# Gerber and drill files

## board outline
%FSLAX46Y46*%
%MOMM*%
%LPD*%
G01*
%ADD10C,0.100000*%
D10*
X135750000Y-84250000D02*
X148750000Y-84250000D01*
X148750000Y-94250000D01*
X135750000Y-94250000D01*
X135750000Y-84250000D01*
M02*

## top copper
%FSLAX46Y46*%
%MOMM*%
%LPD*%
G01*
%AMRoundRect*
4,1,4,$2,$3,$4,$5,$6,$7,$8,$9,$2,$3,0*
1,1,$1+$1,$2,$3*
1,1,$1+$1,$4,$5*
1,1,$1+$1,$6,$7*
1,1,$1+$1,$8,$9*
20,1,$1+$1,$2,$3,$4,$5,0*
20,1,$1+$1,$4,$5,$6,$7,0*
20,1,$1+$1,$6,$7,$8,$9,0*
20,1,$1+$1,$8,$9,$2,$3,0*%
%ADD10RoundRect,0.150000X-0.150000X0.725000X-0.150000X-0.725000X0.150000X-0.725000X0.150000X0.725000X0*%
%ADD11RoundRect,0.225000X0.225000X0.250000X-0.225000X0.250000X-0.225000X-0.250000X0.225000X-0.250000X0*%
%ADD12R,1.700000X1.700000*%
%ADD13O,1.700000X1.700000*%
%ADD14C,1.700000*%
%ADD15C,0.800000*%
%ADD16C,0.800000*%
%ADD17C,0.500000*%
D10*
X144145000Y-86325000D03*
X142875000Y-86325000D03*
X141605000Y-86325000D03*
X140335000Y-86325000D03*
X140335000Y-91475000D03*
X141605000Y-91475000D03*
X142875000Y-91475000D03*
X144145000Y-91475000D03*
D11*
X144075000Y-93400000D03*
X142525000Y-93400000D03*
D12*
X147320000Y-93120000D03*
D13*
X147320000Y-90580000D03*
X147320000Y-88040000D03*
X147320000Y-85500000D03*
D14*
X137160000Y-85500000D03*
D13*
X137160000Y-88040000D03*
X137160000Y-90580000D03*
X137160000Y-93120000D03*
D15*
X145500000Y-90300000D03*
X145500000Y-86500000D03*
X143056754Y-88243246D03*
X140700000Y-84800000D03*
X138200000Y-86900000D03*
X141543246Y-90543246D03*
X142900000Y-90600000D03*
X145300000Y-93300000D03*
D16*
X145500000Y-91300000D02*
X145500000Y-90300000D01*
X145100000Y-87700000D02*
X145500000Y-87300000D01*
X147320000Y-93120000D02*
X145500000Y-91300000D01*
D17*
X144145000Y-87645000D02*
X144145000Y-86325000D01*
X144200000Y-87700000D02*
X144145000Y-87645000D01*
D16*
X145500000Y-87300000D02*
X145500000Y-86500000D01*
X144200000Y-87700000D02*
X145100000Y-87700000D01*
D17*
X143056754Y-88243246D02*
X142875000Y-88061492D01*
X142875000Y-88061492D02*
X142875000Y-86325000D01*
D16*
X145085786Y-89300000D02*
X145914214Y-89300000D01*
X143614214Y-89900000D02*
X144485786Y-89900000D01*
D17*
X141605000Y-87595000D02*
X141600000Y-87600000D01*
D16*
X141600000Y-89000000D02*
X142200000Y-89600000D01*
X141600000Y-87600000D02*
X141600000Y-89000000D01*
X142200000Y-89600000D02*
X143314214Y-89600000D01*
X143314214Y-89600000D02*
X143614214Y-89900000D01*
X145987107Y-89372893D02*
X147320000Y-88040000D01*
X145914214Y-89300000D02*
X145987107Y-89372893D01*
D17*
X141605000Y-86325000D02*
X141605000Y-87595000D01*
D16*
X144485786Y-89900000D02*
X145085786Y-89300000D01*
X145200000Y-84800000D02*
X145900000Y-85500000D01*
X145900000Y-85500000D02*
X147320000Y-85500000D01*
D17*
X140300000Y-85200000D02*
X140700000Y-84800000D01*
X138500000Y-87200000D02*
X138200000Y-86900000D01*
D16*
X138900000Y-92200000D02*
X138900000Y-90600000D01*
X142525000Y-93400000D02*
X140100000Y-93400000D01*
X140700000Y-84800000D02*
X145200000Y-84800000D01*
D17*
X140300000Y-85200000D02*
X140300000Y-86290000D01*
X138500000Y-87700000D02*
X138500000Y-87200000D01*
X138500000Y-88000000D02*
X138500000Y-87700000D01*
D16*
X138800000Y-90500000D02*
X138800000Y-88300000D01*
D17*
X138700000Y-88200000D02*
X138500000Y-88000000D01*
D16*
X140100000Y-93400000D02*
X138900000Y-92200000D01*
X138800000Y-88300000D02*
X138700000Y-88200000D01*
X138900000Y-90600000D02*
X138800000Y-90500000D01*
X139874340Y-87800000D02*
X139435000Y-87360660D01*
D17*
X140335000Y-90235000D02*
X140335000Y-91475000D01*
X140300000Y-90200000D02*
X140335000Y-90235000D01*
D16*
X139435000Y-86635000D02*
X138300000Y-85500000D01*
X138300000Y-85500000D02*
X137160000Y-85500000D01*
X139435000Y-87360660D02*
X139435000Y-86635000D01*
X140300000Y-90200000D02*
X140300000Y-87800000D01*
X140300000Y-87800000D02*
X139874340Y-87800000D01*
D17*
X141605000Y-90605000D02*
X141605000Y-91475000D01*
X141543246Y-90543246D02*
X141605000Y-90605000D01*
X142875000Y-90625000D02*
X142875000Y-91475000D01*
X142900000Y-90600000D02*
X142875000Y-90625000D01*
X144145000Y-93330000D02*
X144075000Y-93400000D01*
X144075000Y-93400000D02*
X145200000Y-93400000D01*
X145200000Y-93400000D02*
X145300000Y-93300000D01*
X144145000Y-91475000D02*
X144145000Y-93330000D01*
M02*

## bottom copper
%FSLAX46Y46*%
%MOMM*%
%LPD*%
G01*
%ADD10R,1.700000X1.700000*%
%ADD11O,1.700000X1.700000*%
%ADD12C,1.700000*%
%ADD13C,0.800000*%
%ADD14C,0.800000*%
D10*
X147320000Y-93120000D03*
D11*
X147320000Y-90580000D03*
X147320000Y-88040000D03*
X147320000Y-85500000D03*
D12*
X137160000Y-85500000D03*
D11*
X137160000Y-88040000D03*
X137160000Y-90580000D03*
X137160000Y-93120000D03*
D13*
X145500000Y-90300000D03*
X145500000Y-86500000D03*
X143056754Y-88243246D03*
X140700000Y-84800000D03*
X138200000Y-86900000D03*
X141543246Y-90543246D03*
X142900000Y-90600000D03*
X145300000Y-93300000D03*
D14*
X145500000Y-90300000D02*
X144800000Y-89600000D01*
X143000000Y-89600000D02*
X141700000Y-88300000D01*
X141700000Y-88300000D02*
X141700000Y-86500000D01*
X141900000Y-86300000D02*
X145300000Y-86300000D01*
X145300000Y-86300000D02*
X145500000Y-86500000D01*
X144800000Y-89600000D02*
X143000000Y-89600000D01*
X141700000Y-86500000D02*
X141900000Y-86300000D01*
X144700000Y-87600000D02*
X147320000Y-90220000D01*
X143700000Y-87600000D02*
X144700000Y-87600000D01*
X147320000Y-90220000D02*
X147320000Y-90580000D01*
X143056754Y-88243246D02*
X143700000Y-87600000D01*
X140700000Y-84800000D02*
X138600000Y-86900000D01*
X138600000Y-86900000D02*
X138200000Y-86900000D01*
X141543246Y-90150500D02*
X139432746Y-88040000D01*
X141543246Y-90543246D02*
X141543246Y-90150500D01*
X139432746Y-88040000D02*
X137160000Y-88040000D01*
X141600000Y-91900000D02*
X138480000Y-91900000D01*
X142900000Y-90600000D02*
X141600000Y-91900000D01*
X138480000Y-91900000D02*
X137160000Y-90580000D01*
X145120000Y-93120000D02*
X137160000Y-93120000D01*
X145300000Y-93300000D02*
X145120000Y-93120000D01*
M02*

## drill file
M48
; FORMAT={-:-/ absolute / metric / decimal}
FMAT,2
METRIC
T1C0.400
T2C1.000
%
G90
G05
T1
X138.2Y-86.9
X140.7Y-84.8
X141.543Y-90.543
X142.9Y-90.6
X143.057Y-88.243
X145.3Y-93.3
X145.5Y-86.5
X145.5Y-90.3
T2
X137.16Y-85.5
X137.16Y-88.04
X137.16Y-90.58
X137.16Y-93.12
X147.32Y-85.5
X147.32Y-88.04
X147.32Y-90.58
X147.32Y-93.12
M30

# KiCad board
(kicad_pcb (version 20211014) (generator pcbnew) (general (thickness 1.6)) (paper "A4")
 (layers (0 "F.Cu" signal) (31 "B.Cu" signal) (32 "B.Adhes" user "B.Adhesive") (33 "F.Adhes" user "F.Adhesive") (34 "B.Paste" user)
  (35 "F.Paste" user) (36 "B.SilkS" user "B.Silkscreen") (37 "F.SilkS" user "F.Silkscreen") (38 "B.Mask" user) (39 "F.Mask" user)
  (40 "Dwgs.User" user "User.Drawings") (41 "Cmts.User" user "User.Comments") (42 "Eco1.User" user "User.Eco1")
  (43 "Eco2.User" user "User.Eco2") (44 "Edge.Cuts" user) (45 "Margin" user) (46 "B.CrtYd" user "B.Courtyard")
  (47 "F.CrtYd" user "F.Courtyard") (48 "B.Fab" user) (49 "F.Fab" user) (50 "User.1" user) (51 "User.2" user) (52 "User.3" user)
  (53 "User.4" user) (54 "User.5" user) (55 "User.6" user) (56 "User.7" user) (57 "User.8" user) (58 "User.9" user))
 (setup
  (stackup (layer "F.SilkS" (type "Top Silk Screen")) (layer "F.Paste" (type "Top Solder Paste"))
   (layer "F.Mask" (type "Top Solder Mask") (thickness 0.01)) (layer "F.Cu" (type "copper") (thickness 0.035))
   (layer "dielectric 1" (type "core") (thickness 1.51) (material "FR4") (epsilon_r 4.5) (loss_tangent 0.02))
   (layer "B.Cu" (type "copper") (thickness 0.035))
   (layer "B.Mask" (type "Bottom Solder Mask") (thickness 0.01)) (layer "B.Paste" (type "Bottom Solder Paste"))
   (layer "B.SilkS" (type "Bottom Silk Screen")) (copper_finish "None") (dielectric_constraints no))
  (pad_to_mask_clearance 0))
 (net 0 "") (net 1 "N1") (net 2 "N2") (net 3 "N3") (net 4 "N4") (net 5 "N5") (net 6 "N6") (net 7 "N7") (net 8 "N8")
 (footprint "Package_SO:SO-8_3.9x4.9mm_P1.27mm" (layer "F.Cu") (at 142.24 88.9 -90)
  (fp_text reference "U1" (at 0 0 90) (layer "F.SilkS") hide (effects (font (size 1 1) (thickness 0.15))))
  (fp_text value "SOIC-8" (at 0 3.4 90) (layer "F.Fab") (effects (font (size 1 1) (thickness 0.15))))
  (pad "1" smd roundrect (at -2.575 -1.905 270) (size 1.75 0.6) (layers "F.Cu" "F.Paste" "F.Mask") (roundrect_rratio 0.25) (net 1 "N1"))
  (pad "2" smd roundrect (at -2.575 -0.635 270) (size 1.75 0.6) (layers "F.Cu" "F.Paste" "F.Mask") (roundrect_rratio 0.25) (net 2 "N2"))
  (pad "3" smd roundrect (at -2.575 0.635 270) (size 1.75 0.6) (layers "F.Cu" "F.Paste" "F.Mask") (roundrect_rratio 0.25) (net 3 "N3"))
  (pad "4" smd roundrect (at -2.575 1.905 270) (size 1.75 0.6) (layers "F.Cu" "F.Paste" "F.Mask") (roundrect_rratio 0.25) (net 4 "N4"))
  (pad "5" smd roundrect (at 2.575 1.905 270) (size 1.75 0.6) (layers "F.Cu" "F.Paste" "F.Mask") (roundrect_rratio 0.25) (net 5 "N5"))
  (pad "6" smd roundrect (at 2.575 0.635 270) (size 1.75 0.6) (layers "F.Cu" "F.Paste" "F.Mask") (roundrect_rratio 0.25) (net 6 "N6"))
  (pad "7" smd roundrect (at 2.575 -0.635 270) (size 1.75 0.6) (layers "F.Cu" "F.Paste" "F.Mask") (roundrect_rratio 0.25) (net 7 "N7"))
  (pad "8" smd roundrect (at 2.575 -1.905 270) (size 1.75 0.6) (layers "F.Cu" "F.Paste" "F.Mask") (roundrect_rratio 0.25) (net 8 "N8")))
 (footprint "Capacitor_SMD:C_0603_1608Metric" (layer "F.Cu") (at 143.3 93.4 180)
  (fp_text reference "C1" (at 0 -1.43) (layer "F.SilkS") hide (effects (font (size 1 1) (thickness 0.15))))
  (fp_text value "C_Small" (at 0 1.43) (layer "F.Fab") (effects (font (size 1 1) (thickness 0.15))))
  (pad "1" smd roundrect (at -0.775 0 180) (size 0.9 0.95) (layers "F.Cu" "F.Paste" "F.Mask") (roundrect_rratio 0.25) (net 8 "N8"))
  (pad "2" smd roundrect (at 0.775 0 180) (size 0.9 0.95) (layers "F.Cu" "F.Paste" "F.Mask") (roundrect_rratio 0.25) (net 4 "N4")))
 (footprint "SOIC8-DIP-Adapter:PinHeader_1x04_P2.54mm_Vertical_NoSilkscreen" (layer "B.Cu") (at 147.32 93.12)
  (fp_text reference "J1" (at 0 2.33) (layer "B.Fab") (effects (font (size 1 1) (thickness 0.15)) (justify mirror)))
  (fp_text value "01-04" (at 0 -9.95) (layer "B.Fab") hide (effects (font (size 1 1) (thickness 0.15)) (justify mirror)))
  (pad "1" thru_hole rect (at 0 0) (size 1.7 1.7) (drill 1) (layers *.Cu *.Mask) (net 1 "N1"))
  (pad "2" thru_hole oval (at 0 -2.54) (size 1.7 1.7) (drill 1) (layers *.Cu *.Mask) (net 2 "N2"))
  (pad "3" thru_hole oval (at 0 -5.08) (size 1.7 1.7) (drill 1) (layers *.Cu *.Mask) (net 3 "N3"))
  (pad "4" thru_hole oval (at 0 -7.62) (size 1.7 1.7) (drill 1) (layers *.Cu *.Mask) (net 4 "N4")))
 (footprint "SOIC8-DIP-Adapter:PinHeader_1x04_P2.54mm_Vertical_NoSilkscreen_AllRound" (layer "B.Cu") (at 137.16 85.5 180)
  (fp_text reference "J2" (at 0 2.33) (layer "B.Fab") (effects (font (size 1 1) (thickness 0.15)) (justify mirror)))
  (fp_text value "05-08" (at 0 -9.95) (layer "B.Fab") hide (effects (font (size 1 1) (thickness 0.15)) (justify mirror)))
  (pad "1" thru_hole circle (at 0 0 180) (size 1.7 1.7) (drill 1) (layers *.Cu *.Mask) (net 5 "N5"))
  (pad "2" thru_hole oval (at 0 -2.54 180) (size 1.7 1.7) (drill 1) (layers *.Cu *.Mask) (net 6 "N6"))
  (pad "3" thru_hole oval (at 0 -5.08 180) (size 1.7 1.7) (drill 1) (layers *.Cu *.Mask) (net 7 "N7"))
  (pad "4" thru_hole oval (at 0 -7.62 180) (size 1.7 1.7) (drill 1) (layers *.Cu *.Mask) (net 8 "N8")))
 (gr_rect (start 135.75 84.25) (end 148.75 94.25) (layer "Edge.Cuts") (width 0.1) (fill none))
 (segment (start 145.5 91.3) (end 145.5 90.3) (width 0.8) (layer "F.Cu") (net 1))
 (segment (start 145.1 87.7) (end 145.5 87.3) (width 0.8) (layer "F.Cu") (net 1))
 (segment (start 147.32 93.12) (end 145.5 91.3) (width 0.8) (layer "F.Cu") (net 1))
 (segment (start 144.145 87.645) (end 144.145 86.325) (width 0.5) (layer "F.Cu") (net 1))
 (segment (start 144.2 87.7) (end 144.145 87.645) (width 0.5) (layer "F.Cu") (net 1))
 (segment (start 145.5 87.3) (end 145.5 86.5) (width 0.8) (layer "F.Cu") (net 1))
 (segment (start 144.2 87.7) (end 145.1 87.7) (width 0.8) (layer "F.Cu") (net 1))
 (via (at 145.5 90.3) (size 0.8) (drill 0.4) (layers "F.Cu" "B.Cu") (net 1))
 (via (at 145.5 86.5) (size 0.8) (drill 0.4) (layers "F.Cu" "B.Cu") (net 1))
 (segment (start 145.5 90.3) (end 144.8 89.6) (width 0.8) (layer "B.Cu") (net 1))
 (segment (start 143 89.6) (end 141.7 88.3) (width 0.8) (layer "B.Cu") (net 1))
 (segment (start 141.7 88.3) (end 141.7 86.5) (width 0.8) (layer "B.Cu") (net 1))
 (segment (start 141.9 86.3) (end 145.3 86.3) (width 0.8) (layer "B.Cu") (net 1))
 (segment (start 145.3 86.3) (end 145.5 86.5) (width 0.8) (layer "B.Cu") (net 1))
 (segment (start 144.8 89.6) (end 143 89.6) (width 0.8) (layer "B.Cu") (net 1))
 (segment (start 141.7 86.5) (end 141.9 86.3) (width 0.8) (layer "B.Cu") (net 1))
 (segment (start 143.056754 88.243246) (end 142.875 88.061492) (width 0.5) (layer "F.Cu") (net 2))
 (segment (start 142.875 88.061492) (end 142.875 86.325) (width 0.5) (layer "F.Cu") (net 2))
 (via (at 143.056754 88.243246) (size 0.8) (drill 0.4) (layers "F.Cu" "B.Cu") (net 2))
 (segment (start 144.7 87.6) (end 147.32 90.22) (width 0.8) (layer "B.Cu") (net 2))
 (segment (start 143.7 87.6) (end 144.7 87.6) (width 0.8) (layer "B.Cu") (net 2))
 (segment (start 147.32 90.22) (end 147.32 90.58) (width 0.8) (layer "B.Cu") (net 2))
 (segment (start 143.056754 88.243246) (end 143.7 87.6) (width 0.8) (layer "B.Cu") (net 2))
 (segment (start 145.085786 89.3) (end 145.914214 89.3) (width 0.8) (layer "F.Cu") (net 3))
 (segment (start 143.614214 89.9) (end 144.485786 89.9) (width 0.8) (layer "F.Cu") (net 3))
 (segment (start 141.605 87.595) (end 141.6 87.6) (width 0.5) (layer "F.Cu") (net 3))
 (segment (start 141.6 89) (end 142.2 89.6) (width 0.8) (layer "F.Cu") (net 3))
 (segment (start 141.6 87.6) (end 141.6 89) (width 0.8) (layer "F.Cu") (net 3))
 (segment (start 142.2 89.6) (end 143.314214 89.6) (width 0.8) (layer "F.Cu") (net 3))
 (segment (start 143.314214 89.6) (end 143.614214 89.9) (width 0.8) (layer "F.Cu") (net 3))
 (segment (start 145.987107 89.372893) (end 147.32 88.04) (width 0.8) (layer "F.Cu") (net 3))
 (segment (start 145.914214 89.3) (end 145.987107 89.372893) (width 0.8) (layer "F.Cu") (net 3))
 (segment (start 141.605 86.325) (end 141.605 87.595) (width 0.5) (layer "F.Cu") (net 3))
 (segment (start 144.485786 89.9) (end 145.085786 89.3) (width 0.8) (layer "F.Cu") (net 3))
 (segment (start 145.2 84.8) (end 145.9 85.5) (width 0.8) (layer "F.Cu") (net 4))
 (segment (start 145.9 85.5) (end 147.32 85.5) (width 0.8) (layer "F.Cu") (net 4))
 (segment (start 140.3 85.2) (end 140.7 84.8) (width 0.5) (layer "F.Cu") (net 4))
 (segment (start 138.5 87.2) (end 138.2 86.9) (width 0.5) (layer "F.Cu") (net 4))
 (segment (start 138.9 92.2) (end 138.9 90.6) (width 0.8) (layer "F.Cu") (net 4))
 (segment (start 142.525 93.4) (end 140.1 93.4) (width 0.8) (layer "F.Cu") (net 4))
 (segment (start 140.7 84.8) (end 145.2 84.8) (width 0.8) (layer "F.Cu") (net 4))
 (segment (start 140.3 85.2) (end 140.3 86.29) (width 0.5) (layer "F.Cu") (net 4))
 (segment (start 138.5 87.7) (end 138.5 87.2) (width 0.5) (layer "F.Cu") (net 4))
 (segment (start 138.5 88) (end 138.5 87.7) (width 0.5) (layer "F.Cu") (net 4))
 (segment (start 138.8 90.5) (end 138.8 88.3) (width 0.8) (layer "F.Cu") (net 4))
 (segment (start 138.7 88.2) (end 138.5 88) (width 0.5) (layer "F.Cu") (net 4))
 (segment (start 140.1 93.4) (end 138.9 92.2) (width 0.8) (layer "F.Cu") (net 4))
 (segment (start 138.8 88.3) (end 138.7 88.2) (width 0.8) (layer "F.Cu") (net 4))
 (segment (start 138.9 90.6) (end 138.8 90.5) (width 0.8) (layer "F.Cu") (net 4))
 (via (at 140.7 84.8) (size 0.8) (drill 0.4) (layers "F.Cu" "B.Cu") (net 4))
 (via (at 138.2 86.9) (size 0.8) (drill 0.4) (layers "F.Cu" "B.Cu") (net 4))
 (segment (start 140.7 84.8) (end 138.6 86.9) (width 0.8) (layer "B.Cu") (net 4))
 (segment (start 138.6 86.9) (end 138.2 86.9) (width 0.8) (layer "B.Cu") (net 4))
 (segment (start 139.87434 87.8) (end 139.435 87.36066) (width 0.8) (layer "F.Cu") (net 5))
 (segment (start 140.335 90.235) (end 140.335 91.475) (width 0.5) (layer "F.Cu") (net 5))
 (segment (start 140.3 90.2) (end 140.335 90.235) (width 0.5) (layer "F.Cu") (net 5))
 (segment (start 139.435 86.635) (end 138.3 85.5) (width 0.8) (layer "F.Cu") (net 5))
 (segment (start 138.3 85.5) (end 137.16 85.5) (width 0.8) (layer "F.Cu") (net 5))
 (segment (start 139.435 87.36066) (end 139.435 86.635) (width 0.8) (layer "F.Cu") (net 5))
 (segment (start 140.3 90.2) (end 140.3 87.8) (width 0.8) (layer "F.Cu") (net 5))
 (segment (start 140.3 87.8) (end 139.87434 87.8) (width 0.8) (layer "F.Cu") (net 5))
 (segment (start 141.605 90.605) (end 141.605 91.475) (width 0.5) (layer "F.Cu") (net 6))
 (segment (start 141.543246 90.543246) (end 141.605 90.605) (width 0.5) (layer "F.Cu") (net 6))
 (via (at 141.543246 90.543246) (size 0.8) (drill 0.4) (layers "F.Cu" "B.Cu") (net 6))
 (segment (start 141.543246 90.1505) (end 139.432746 88.04) (width 0.8) (layer "B.Cu") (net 6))
 (segment (start 141.543246 90.543246) (end 141.543246 90.1505) (width 0.8) (layer "B.Cu") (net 6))
 (segment (start 139.432746 88.04) (end 137.16 88.04) (width 0.8) (layer "B.Cu") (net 6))
 (segment (start 142.875 90.625) (end 142.875 91.475) (width 0.5) (layer "F.Cu") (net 7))
 (segment (start 142.9 90.6) (end 142.875 90.625) (width 0.5) (layer "F.Cu") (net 7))
 (via (at 142.9 90.6) (size 0.8) (drill 0.4) (layers "F.Cu" "B.Cu") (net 7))
 (segment (start 141.6 91.9) (end 138.48 91.9) (width 0.8) (layer "B.Cu") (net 7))
 (segment (start 142.9 90.6) (end 141.6 91.9) (width 0.8) (layer "B.Cu") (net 7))
 (segment (start 138.48 91.9) (end 137.16 90.58) (width 0.8) (layer "B.Cu") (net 7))
 (segment (start 144.145 93.33) (end 144.075 93.4) (width 0.5) (layer "F.Cu") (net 8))
 (segment (start 144.075 93.4) (end 145.2 93.4) (width 0.5) (layer "F.Cu") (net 8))
 (segment (start 145.2 93.4) (end 145.3 93.3) (width 0.5) (layer "F.Cu") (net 8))
 (segment (start 144.145 91.475) (end 144.145 93.33) (width 0.5) (layer "F.Cu") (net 8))
 (via (at 145.3 93.3) (size 0.8) (drill 0.4) (layers "F.Cu" "B.Cu") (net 8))
 (segment (start 145.12 93.12) (end 137.16 93.12) (width 0.8) (layer "B.Cu") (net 8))
 (segment (start 145.3 93.3) (end 145.12 93.12) (width 0.8) (layer "B.Cu") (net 8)))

